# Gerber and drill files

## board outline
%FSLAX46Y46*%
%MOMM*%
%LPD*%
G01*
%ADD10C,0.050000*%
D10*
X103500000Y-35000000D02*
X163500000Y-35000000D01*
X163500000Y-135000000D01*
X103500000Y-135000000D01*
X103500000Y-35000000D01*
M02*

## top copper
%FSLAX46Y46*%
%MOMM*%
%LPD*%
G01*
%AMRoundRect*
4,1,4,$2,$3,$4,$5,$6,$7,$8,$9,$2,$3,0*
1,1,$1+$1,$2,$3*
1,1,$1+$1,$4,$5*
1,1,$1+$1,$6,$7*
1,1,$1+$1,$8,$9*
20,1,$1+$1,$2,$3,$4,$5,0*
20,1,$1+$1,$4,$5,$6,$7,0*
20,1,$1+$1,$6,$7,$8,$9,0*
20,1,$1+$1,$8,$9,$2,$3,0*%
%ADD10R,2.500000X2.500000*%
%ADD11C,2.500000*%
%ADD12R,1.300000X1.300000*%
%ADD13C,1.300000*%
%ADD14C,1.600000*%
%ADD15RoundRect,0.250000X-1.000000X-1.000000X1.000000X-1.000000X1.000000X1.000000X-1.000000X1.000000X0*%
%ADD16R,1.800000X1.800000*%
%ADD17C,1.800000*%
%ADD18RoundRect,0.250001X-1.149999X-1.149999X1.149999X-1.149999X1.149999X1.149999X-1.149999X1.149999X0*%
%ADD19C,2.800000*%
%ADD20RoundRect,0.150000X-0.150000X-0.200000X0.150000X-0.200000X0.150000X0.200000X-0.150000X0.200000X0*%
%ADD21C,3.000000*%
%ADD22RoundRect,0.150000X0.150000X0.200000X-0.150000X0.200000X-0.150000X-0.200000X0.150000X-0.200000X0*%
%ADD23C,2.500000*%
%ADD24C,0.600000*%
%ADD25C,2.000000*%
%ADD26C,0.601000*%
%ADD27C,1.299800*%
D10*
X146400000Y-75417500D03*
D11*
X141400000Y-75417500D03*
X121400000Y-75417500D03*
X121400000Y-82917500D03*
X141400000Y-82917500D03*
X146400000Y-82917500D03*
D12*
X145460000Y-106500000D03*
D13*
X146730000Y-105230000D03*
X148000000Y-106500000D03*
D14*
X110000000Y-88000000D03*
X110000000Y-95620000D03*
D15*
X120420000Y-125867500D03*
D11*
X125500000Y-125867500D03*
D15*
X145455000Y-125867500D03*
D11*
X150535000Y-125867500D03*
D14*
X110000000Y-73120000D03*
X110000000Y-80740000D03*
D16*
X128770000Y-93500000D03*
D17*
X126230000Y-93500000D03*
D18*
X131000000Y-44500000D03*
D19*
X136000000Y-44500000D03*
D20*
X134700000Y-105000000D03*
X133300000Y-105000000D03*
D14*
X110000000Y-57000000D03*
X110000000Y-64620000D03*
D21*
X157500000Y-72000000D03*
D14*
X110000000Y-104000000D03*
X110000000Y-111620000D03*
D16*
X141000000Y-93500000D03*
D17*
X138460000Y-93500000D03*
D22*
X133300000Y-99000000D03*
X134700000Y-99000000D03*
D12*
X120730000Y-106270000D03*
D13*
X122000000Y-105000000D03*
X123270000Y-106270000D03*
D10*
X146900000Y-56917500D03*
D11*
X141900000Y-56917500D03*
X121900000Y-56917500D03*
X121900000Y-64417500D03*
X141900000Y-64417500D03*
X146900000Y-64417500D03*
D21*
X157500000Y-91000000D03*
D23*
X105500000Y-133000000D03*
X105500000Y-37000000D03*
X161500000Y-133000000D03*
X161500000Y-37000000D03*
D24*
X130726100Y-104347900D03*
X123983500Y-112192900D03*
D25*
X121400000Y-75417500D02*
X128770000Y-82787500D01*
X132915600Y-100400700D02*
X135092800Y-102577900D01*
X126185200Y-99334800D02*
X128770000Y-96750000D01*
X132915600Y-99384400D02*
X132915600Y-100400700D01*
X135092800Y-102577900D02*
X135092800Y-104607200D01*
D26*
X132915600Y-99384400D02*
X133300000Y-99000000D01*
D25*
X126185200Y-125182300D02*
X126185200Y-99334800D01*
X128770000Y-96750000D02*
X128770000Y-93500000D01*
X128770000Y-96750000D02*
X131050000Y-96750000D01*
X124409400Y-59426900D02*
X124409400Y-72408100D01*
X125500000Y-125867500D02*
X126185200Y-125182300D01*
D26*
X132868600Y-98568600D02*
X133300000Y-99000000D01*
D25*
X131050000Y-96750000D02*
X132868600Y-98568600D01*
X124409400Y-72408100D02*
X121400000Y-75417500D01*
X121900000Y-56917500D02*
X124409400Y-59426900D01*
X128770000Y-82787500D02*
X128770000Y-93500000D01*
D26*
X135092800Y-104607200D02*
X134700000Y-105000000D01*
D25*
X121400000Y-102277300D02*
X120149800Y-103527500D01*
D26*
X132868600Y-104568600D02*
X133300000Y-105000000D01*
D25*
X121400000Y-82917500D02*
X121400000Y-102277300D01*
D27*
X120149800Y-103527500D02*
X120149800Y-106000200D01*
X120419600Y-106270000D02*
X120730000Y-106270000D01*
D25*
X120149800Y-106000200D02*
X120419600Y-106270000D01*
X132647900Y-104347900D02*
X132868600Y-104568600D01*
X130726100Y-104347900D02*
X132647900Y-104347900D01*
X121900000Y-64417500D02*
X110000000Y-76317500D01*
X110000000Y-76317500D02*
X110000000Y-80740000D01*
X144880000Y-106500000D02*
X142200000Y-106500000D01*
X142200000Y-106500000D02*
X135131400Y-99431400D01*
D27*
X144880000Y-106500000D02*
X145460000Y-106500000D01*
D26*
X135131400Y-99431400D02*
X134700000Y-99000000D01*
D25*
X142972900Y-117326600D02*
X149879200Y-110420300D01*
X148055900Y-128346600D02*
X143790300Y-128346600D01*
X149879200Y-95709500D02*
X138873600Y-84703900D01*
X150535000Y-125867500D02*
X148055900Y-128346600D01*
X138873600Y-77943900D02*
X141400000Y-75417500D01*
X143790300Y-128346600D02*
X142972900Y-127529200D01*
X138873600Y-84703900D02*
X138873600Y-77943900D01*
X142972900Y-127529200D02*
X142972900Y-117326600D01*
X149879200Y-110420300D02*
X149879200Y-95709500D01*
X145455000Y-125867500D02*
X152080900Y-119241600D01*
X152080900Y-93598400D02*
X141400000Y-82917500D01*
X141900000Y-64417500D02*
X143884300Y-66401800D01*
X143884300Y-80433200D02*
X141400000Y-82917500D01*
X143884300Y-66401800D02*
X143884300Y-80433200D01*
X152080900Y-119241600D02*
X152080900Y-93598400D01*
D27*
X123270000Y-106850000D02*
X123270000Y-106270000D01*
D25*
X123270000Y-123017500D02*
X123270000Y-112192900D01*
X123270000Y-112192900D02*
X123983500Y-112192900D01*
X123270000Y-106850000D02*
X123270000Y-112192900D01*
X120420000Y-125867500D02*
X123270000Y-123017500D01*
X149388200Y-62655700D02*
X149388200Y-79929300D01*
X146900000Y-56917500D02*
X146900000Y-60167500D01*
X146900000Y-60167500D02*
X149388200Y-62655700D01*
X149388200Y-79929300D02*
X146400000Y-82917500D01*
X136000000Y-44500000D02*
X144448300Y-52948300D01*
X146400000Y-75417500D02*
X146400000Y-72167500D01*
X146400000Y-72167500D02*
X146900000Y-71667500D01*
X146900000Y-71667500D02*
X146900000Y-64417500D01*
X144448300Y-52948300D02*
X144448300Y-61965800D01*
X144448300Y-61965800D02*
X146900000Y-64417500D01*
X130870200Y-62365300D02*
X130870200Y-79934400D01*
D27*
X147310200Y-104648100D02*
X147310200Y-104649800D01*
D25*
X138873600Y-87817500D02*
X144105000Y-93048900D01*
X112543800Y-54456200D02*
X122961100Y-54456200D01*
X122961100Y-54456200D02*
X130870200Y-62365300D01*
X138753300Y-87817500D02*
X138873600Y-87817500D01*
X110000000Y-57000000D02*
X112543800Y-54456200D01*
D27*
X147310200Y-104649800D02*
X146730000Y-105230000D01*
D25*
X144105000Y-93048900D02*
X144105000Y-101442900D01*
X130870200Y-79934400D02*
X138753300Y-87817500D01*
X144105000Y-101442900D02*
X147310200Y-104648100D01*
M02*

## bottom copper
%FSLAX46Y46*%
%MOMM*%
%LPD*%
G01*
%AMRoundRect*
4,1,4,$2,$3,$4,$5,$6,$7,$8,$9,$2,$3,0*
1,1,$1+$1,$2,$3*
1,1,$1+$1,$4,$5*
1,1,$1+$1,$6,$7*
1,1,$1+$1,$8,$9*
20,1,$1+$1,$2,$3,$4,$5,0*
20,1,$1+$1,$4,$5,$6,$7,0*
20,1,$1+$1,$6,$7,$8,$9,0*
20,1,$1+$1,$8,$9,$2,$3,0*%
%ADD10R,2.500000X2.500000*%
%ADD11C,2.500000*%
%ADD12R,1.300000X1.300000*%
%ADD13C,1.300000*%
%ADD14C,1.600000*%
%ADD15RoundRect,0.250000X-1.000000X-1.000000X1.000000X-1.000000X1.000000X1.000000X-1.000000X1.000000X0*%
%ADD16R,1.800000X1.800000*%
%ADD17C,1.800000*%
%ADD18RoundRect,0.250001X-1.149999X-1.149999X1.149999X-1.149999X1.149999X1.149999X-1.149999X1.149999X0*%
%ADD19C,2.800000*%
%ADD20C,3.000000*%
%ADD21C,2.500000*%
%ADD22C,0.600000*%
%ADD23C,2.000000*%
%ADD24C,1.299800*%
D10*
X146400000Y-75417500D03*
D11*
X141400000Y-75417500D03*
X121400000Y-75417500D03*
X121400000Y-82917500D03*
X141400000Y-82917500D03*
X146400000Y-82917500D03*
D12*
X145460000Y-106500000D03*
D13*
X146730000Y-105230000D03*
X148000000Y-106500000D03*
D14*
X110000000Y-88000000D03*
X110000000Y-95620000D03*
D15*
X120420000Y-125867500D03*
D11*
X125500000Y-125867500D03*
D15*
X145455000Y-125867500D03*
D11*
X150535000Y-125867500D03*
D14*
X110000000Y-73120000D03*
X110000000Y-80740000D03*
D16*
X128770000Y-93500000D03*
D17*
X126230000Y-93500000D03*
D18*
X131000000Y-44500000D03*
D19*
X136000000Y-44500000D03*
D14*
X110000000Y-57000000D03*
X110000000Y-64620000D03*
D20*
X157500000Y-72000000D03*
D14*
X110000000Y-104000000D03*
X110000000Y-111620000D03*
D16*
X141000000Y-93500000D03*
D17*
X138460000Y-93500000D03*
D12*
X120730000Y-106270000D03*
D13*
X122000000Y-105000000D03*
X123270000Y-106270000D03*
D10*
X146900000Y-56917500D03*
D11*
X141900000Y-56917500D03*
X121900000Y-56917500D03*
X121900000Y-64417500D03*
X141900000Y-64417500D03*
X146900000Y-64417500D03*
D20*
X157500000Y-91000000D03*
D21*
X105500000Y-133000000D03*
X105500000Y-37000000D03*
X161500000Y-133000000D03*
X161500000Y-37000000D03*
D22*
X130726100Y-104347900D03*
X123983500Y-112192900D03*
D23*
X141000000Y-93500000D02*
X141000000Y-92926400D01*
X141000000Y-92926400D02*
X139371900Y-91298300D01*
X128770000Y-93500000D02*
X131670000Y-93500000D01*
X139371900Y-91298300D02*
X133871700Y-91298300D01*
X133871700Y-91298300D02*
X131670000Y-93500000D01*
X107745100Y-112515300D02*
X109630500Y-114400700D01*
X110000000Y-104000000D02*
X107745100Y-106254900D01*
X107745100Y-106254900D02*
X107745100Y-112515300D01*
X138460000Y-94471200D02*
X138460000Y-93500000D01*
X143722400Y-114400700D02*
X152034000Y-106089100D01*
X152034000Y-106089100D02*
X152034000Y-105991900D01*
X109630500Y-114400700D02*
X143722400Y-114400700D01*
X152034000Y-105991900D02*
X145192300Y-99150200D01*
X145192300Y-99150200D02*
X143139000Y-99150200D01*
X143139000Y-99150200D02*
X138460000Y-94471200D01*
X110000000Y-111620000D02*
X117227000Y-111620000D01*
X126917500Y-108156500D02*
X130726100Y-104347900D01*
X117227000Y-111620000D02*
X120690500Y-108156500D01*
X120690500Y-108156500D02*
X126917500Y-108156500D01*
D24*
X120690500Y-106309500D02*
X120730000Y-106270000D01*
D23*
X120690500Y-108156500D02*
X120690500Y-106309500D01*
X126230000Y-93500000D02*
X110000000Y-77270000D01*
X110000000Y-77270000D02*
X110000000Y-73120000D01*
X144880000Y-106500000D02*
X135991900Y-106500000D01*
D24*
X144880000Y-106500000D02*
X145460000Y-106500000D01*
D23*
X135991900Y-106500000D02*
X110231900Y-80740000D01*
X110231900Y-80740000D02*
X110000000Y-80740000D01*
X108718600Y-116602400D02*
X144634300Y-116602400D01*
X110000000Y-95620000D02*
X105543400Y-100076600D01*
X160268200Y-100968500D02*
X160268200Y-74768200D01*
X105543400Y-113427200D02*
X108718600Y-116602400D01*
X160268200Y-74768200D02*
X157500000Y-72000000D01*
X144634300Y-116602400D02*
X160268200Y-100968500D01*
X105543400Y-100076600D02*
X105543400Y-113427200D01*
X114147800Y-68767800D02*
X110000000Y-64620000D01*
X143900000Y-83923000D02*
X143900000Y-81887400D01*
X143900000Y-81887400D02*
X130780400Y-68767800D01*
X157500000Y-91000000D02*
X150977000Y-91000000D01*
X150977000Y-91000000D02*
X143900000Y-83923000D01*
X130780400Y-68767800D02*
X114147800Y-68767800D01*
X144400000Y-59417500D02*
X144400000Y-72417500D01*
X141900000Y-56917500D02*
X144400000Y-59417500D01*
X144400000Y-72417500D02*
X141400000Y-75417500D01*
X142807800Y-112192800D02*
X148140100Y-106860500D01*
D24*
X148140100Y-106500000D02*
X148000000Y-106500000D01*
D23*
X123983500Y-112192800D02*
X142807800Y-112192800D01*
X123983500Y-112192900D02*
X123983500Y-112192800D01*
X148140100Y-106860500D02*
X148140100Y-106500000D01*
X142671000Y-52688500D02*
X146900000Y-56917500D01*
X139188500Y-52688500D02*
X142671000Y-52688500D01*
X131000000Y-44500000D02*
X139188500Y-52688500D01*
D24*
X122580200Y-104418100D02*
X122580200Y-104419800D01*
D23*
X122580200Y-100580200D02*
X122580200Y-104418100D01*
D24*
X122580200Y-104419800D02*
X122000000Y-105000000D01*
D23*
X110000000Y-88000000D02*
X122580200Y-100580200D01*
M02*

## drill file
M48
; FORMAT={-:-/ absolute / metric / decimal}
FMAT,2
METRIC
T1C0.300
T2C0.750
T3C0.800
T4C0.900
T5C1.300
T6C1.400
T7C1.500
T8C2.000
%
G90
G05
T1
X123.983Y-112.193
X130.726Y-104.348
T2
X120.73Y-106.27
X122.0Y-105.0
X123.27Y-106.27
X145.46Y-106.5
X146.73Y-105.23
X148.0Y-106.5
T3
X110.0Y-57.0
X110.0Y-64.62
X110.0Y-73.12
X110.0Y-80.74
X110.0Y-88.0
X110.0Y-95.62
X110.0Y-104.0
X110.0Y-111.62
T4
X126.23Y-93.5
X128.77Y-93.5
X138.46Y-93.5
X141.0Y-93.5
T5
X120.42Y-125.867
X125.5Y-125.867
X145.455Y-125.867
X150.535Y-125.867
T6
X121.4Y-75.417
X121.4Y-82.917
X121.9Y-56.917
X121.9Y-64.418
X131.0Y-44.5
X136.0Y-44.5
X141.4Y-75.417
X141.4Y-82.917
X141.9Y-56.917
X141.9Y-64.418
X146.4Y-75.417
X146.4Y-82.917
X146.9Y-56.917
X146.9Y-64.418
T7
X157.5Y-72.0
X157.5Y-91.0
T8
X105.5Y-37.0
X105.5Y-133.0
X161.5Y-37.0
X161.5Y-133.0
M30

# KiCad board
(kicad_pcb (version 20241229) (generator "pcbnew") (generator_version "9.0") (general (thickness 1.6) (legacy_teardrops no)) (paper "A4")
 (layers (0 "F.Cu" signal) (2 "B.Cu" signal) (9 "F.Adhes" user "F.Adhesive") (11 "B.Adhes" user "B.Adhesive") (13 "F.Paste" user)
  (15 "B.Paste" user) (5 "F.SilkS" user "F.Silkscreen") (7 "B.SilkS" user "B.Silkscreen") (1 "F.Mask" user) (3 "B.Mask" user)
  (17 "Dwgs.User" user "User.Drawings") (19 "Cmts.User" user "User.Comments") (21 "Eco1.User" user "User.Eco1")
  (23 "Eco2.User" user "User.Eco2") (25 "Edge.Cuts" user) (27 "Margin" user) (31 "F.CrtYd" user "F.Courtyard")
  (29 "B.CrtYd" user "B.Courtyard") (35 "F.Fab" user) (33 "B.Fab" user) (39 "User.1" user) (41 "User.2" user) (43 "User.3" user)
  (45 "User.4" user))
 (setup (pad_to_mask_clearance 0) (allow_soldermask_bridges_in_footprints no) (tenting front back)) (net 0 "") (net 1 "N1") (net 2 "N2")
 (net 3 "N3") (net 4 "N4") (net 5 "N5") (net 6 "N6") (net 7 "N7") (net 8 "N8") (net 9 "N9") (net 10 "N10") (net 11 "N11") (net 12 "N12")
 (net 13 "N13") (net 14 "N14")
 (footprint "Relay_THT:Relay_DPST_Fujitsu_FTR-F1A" (layer "F.Cu") (at 146.4 75.4175 -90)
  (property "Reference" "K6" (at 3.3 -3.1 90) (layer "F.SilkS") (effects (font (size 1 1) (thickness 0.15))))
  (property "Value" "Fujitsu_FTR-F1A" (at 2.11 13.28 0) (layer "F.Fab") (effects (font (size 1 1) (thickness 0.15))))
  (pad "1" thru_hole rect (at 0 0 180) (size 2.5 2.5) (drill 1.4) (layers "*.Cu" "*.Mask") (remove_unused_layers no) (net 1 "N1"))
  (pad "2" thru_hole circle (at 0 5 180) (size 2.5 2.5) (drill 1.4) (layers "*.Cu" "*.Mask") (remove_unused_layers no) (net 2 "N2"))
  (pad "4" thru_hole circle (at 0 25 180) (size 2.5 2.5) (drill 1.4) (layers "*.Cu" "*.Mask") (remove_unused_layers no) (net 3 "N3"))
  (pad "5" thru_hole circle (at 7.5 25 180) (size 2.5 2.5) (drill 1.4) (layers "*.Cu" "*.Mask") (remove_unused_layers no) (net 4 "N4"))
  (pad "7" thru_hole circle (at 7.5 5 180) (size 2.5 2.5) (drill 1.4) (layers "*.Cu" "*.Mask") (remove_unused_layers no) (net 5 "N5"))
  (pad "8" thru_hole circle (at 7.5 0 180) (size 2.5 2.5) (drill 1.4) (layers "*.Cu" "*.Mask") (remove_unused_layers no) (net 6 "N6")))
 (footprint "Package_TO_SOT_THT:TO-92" (layer "F.Cu") (at 145.46 106.5)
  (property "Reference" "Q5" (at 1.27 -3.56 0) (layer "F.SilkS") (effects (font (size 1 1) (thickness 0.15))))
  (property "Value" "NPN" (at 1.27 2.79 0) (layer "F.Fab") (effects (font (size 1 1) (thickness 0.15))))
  (pad "1" thru_hole rect (at 0 0) (size 1.3 1.3) (drill 0.75) (layers "*.Cu" "*.Mask") (remove_unused_layers no) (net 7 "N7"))
  (pad "2" thru_hole circle (at 1.27 -1.27) (size 1.3 1.3) (drill 0.75) (layers "*.Cu" "*.Mask") (remove_unused_layers no) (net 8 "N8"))
  (pad "3" thru_hole circle (at 2.54 0) (size 1.3 1.3) (drill 0.75) (layers "*.Cu" "*.Mask") (remove_unused_layers no) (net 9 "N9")))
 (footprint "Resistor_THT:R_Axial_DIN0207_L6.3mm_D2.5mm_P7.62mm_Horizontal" (layer "F.Cu") (at 110 88 -90)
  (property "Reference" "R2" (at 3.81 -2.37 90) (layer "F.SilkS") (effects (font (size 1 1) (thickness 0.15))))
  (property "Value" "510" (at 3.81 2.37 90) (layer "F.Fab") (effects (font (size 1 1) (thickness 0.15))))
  (pad "1" thru_hole circle (at 0 0 270) (size 1.6 1.6) (drill 0.8) (layers "*.Cu" "*.Mask") (remove_unused_layers no) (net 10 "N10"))
  (pad "2" thru_hole circle (at 7.62 0 270) (size 1.6 1.6) (drill 0.8) (layers "*.Cu" "*.Mask") (remove_unused_layers no) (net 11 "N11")))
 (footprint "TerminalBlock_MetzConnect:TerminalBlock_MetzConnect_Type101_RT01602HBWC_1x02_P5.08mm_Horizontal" (layer "F.Cu")
  (at 120.42 125.8675)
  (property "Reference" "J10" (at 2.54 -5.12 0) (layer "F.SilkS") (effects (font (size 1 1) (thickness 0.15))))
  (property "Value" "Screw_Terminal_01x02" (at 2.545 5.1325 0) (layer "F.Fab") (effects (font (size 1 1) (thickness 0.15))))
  (pad "1" thru_hole roundrect (at 0 0) (size 2.5 2.5) (drill 1.3) (layers "*.Cu" "*.Mask") (remove_unused_layers no) (roundrect_rratio 0.1)
   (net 9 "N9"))
  (pad "2" thru_hole circle (at 5.08 0) (size 2.5 2.5) (drill 1.3) (layers "*.Cu" "*.Mask") (remove_unused_layers no) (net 3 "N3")))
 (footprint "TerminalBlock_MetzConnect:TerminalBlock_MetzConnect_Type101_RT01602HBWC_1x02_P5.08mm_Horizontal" (layer "F.Cu")
  (at 145.455 125.8675)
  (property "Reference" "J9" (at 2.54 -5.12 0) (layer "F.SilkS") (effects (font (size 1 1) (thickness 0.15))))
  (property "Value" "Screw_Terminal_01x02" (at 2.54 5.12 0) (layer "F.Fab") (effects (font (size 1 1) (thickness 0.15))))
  (pad "1" thru_hole roundrect (at 0 0) (size 2.5 2.5) (drill 1.3) (layers "*.Cu" "*.Mask") (remove_unused_layers no) (roundrect_rratio 0.1)
   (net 5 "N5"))
  (pad "2" thru_hole circle (at 5.08 0) (size 2.5 2.5) (drill 1.3) (layers "*.Cu" "*.Mask") (remove_unused_layers no) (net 2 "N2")))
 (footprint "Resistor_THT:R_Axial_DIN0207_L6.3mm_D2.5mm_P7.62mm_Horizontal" (layer "F.Cu") (at 110 73.12 -90)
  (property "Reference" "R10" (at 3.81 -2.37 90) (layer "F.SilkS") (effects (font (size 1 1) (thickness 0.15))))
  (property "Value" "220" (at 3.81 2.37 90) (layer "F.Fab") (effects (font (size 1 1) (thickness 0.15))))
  (pad "1" thru_hole circle (at 0 0 270) (size 1.6 1.6) (drill 0.8) (layers "*.Cu" "*.Mask") (remove_unused_layers no) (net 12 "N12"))
  (pad "2" thru_hole circle (at 7.62 0 270) (size 1.6 1.6) (drill 0.8) (layers "*.Cu" "*.Mask") (remove_unused_layers no) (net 7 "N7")))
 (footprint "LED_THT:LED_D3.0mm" (layer "F.Cu") (at 128.77 93.5 180)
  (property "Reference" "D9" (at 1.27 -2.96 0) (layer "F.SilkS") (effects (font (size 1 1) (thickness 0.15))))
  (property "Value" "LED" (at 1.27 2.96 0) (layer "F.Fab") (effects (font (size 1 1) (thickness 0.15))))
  (pad "1" thru_hole rect (at 0 0 180) (size 1.8 1.8) (drill 0.9) (layers "*.Cu" "*.Mask") (remove_unused_layers no) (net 3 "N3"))
  (pad "2" thru_hole circle (at 2.54 0 180) (size 1.8 1.8) (drill 0.9) (layers "*.Cu" "*.Mask") (remove_unused_layers no) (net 12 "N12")))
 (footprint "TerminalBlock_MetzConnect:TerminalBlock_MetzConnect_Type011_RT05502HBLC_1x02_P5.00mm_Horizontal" (layer "F.Cu") (at 131 44.5)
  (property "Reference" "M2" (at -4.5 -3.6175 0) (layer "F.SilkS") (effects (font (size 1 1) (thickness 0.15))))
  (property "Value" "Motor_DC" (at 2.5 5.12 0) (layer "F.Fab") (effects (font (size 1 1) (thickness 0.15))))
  (pad "1" thru_hole roundrect (at 0 0) (size 2.8 2.8) (drill 1.4) (layers "*.Cu" "*.Mask") (remove_unused_layers no)
   (roundrect_rratio 0.089286) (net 6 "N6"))
  (pad "2" thru_hole circle (at 5 0) (size 2.8 2.8) (drill 1.4) (layers "*.Cu" "*.Mask") (remove_unused_layers no) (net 1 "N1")))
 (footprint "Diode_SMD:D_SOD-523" (layer "F.Cu") (at 134 105 180)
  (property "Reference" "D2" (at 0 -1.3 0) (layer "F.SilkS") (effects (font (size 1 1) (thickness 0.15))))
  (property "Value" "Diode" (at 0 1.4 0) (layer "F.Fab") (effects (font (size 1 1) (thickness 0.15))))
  (pad "1" smd roundrect (at -0.7 0) (size 0.6 0.7) (layers "F.Cu" "F.Mask" "F.Paste") (roundrect_rratio 0.25) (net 3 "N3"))
  (pad "2" smd roundrect (at 0.7 0) (size 0.6 0.7) (layers "F.Cu" "F.Mask" "F.Paste") (roundrect_rratio 0.25) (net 4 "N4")))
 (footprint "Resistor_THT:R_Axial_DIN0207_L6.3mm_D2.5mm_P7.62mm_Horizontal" (layer "F.Cu") (at 110 57 -90)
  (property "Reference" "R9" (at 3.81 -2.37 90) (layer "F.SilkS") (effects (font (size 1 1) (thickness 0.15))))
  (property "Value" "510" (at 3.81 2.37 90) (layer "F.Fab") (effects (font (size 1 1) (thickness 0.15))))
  (pad "1" thru_hole circle (at 0 0 270) (size 1.6 1.6) (drill 0.8) (layers "*.Cu" "*.Mask") (remove_unused_layers no) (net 8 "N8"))
  (pad "2" thru_hole circle (at 7.62 0 270) (size 1.6 1.6) (drill 0.8) (layers "*.Cu" "*.Mask") (remove_unused_layers no) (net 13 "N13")))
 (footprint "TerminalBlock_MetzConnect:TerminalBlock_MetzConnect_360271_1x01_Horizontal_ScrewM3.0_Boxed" (layer "F.Cu") (at 157.5 72 90)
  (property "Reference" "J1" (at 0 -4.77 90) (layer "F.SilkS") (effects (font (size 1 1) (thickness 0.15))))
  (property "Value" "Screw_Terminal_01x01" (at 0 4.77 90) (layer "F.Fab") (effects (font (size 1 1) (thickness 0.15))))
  (pad "1" thru_hole circle (at 0 0 90) (size 3 3) (drill 1.5) (layers "*.Cu" "*.Mask") (remove_unused_layers no) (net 11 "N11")))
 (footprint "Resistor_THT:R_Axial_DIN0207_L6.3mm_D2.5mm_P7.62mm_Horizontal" (layer "F.Cu") (at 110 104 -90)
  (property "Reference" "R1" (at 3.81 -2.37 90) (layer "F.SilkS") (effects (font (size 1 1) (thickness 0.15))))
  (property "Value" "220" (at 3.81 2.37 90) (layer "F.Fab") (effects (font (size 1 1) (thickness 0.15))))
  (pad "1" thru_hole circle (at 0 0 270) (size 1.6 1.6) (drill 0.8) (layers "*.Cu" "*.Mask") (remove_unused_layers no) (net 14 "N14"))
  (pad "2" thru_hole circle (at 7.62 0 270) (size 1.6 1.6) (drill 0.8) (layers "*.Cu" "*.Mask") (remove_unused_layers no) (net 4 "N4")))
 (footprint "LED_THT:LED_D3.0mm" (layer "F.Cu") (at 141 93.5 180)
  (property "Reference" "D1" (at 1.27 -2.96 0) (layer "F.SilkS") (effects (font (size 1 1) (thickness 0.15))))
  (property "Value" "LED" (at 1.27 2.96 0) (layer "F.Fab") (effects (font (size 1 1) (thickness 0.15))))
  (pad "1" thru_hole rect (at 0 0 180) (size 1.8 1.8) (drill 0.9) (layers "*.Cu" "*.Mask") (remove_unused_layers no) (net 3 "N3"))
  (pad "2" thru_hole circle (at 2.54 0 180) (size 1.8 1.8) (drill 0.9) (layers "*.Cu" "*.Mask") (remove_unused_layers no) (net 14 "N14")))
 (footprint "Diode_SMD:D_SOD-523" (layer "F.Cu") (at 134 99)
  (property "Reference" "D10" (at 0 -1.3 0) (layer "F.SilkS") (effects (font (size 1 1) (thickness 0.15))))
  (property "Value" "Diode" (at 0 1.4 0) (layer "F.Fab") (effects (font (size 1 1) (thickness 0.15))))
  (pad "1" smd roundrect (at -0.7 0 180) (size 0.6 0.7) (layers "F.Cu" "F.Mask" "F.Paste") (roundrect_rratio 0.25) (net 3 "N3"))
  (pad "2" smd roundrect (at 0.7 0 180) (size 0.6 0.7) (layers "F.Cu" "F.Mask" "F.Paste") (roundrect_rratio 0.25) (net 7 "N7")))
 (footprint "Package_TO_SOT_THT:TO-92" (layer "F.Cu") (at 120.73 106.27)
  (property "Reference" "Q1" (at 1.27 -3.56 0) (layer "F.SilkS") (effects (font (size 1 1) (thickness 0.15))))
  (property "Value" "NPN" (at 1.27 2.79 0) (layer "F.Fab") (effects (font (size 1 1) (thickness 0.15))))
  (pad "1" thru_hole rect (at 0 0) (size 1.3 1.3) (drill 0.75) (layers "*.Cu" "*.Mask") (remove_unused_layers no) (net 4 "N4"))
  (pad "2" thru_hole circle (at 1.27 -1.27) (size 1.3 1.3) (drill 0.75) (layers "*.Cu" "*.Mask") (remove_unused_layers no) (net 10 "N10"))
  (pad "3" thru_hole circle (at 2.54 0) (size 1.3 1.3) (drill 0.75) (layers "*.Cu" "*.Mask") (remove_unused_layers no) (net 9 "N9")))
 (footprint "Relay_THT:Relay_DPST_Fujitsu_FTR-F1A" (layer "F.Cu") (at 146.9 56.9175 -90)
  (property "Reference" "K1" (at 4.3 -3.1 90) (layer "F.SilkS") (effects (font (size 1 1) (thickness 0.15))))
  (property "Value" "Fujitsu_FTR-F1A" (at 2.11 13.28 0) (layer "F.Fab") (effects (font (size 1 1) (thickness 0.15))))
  (pad "1" thru_hole rect (at 0 0 180) (size 2.5 2.5) (drill 1.4) (layers "*.Cu" "*.Mask") (remove_unused_layers no) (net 6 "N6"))
  (pad "2" thru_hole circle (at 0 5 180) (size 2.5 2.5) (drill 1.4) (layers "*.Cu" "*.Mask") (remove_unused_layers no) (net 2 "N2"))
  (pad "4" thru_hole circle (at 0 25 180) (size 2.5 2.5) (drill 1.4) (layers "*.Cu" "*.Mask") (remove_unused_layers no) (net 3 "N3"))
  (pad "5" thru_hole circle (at 7.5 25 180) (size 2.5 2.5) (drill 1.4) (layers "*.Cu" "*.Mask") (remove_unused_layers no) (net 7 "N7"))
  (pad "7" thru_hole circle (at 7.5 5 180) (size 2.5 2.5) (drill 1.4) (layers "*.Cu" "*.Mask") (remove_unused_layers no) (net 5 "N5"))
  (pad "8" thru_hole circle (at 7.5 0 180) (size 2.5 2.5) (drill 1.4) (layers "*.Cu" "*.Mask") (remove_unused_layers no) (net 1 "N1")))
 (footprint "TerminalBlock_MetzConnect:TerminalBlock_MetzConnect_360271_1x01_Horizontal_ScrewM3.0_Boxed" (layer "F.Cu") (at 157.5 91 90)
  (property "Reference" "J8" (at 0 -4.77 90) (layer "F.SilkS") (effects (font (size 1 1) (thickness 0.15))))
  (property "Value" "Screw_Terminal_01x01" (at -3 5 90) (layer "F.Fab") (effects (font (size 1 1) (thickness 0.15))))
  (pad "1" thru_hole circle (at 0 0 90) (size 3 3) (drill 1.5) (layers "*.Cu" "*.Mask") (remove_unused_layers no) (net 13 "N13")))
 (gr_rect (start 103.5 35) (end 163.5 135) (stroke (width 0.05) (type default)) (fill no) (layer "Edge.Cuts"))
 (via (at 105.5 133) (size 2.5) (drill 2) (layers "F.Cu" "B.Cu") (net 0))
 (via (at 105.5 37) (size 2.5) (drill 2) (layers "F.Cu" "B.Cu") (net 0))
 (via (at 161.5 133) (size 2.5) (drill 2) (layers "F.Cu" "B.Cu") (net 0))
 (via (at 161.5 37) (size 2.5) (drill 2) (layers "F.Cu" "B.Cu") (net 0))
 (segment (start 121.4 75.4175) (end 128.77 82.7875) (width 2) (layer "F.Cu") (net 3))
 (segment (start 132.9156 100.4007) (end 135.0928 102.5779) (width 2) (layer "F.Cu") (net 3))
 (segment (start 126.1852 99.3348) (end 128.77 96.75) (width 2) (layer "F.Cu") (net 3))
 (segment (start 132.9156 99.3844) (end 132.9156 100.4007) (width 2) (layer "F.Cu") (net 3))
 (segment (start 135.0928 102.5779) (end 135.0928 104.6072) (width 2) (layer "F.Cu") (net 3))
 (segment (start 132.9156 99.3844) (end 133.3 99) (width 0.601) (layer "F.Cu") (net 3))
 (segment (start 126.1852 125.1823) (end 126.1852 99.3348) (width 2) (layer "F.Cu") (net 3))
 (segment (start 128.77 96.75) (end 128.77 93.5) (width 2) (layer "F.Cu") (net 3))
 (segment (start 128.77 96.75) (end 131.05 96.75) (width 2) (layer "F.Cu") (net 3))
 (segment (start 124.4094 59.4269) (end 124.4094 72.4081) (width 2) (layer "F.Cu") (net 3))
 (segment (start 125.5 125.8675) (end 126.1852 125.1823) (width 2) (layer "F.Cu") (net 3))
 (segment (start 132.8686 98.5686) (end 133.3 99) (width 0.601) (layer "F.Cu") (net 3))
 (segment (start 131.05 96.75) (end 132.8686 98.5686) (width 2) (layer "F.Cu") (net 3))
 (segment (start 124.4094 72.4081) (end 121.4 75.4175) (width 2) (layer "F.Cu") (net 3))
 (segment (start 121.9 56.9175) (end 124.4094 59.4269) (width 2) (layer "F.Cu") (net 3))
 (segment (start 128.77 82.7875) (end 128.77 93.5) (width 2) (layer "F.Cu") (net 3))
 (segment (start 135.0928 104.6072) (end 134.7 105) (width 0.601) (layer "F.Cu") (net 3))
 (segment (start 141 93.5) (end 141 92.9264) (width 2) (layer "B.Cu") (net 3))
 (segment (start 141 92.9264) (end 139.3719 91.2983) (width 2) (layer "B.Cu") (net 3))
 (segment (start 128.77 93.5) (end 131.67 93.5) (width 2) (layer "B.Cu") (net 3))
 (segment (start 139.3719 91.2983) (end 133.8717 91.2983) (width 2) (layer "B.Cu") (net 3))
 (segment (start 133.8717 91.2983) (end 131.67 93.5) (width 2) (layer "B.Cu") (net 3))
 (segment (start 107.7451 112.5153) (end 109.6305 114.4007) (width 2) (layer "B.Cu") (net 14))
 (segment (start 110 104) (end 107.7451 106.2549) (width 2) (layer "B.Cu") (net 14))
 (segment (start 107.7451 106.2549) (end 107.7451 112.5153) (width 2) (layer "B.Cu") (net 14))
 (segment (start 138.46 94.4712) (end 138.46 93.5) (width 2) (layer "B.Cu") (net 14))
 (segment (start 143.7224 114.4007) (end 152.034 106.0891) (width 2) (layer "B.Cu") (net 14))
 (segment (start 152.034 106.0891) (end 152.034 105.9919) (width 2) (layer "B.Cu") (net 14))
 (segment (start 109.6305 114.4007) (end 143.7224 114.4007) (width 2) (layer "B.Cu") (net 14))
 (segment (start 152.034 105.9919) (end 145.1923 99.1502) (width 2) (layer "B.Cu") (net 14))
 (segment (start 145.1923 99.1502) (end 143.139 99.1502) (width 2) (layer "B.Cu") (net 14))
 (segment (start 143.139 99.1502) (end 138.46 94.4712) (width 2) (layer "B.Cu") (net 14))
 (segment (start 121.4 102.2773) (end 120.1498 103.5275) (width 2) (layer "F.Cu") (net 4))
 (segment (start 132.8686 104.5686) (end 133.3 105) (width 0.601) (layer "F.Cu") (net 4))
 (segment (start 121.4 82.9175) (end 121.4 102.2773) (width 2) (layer "F.Cu") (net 4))
 (segment (start 120.1498 103.5275) (end 120.1498 106.0002) (width 1.2998) (layer "F.Cu") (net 4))
 (segment (start 120.4196 106.27) (end 120.73 106.27) (width 1.2998) (layer "F.Cu") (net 4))
 (segment (start 120.1498 106.0002) (end 120.4196 106.27) (width 2) (layer "F.Cu") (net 4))
 (segment (start 132.6479 104.3479) (end 132.8686 104.5686) (width 2) (layer "F.Cu") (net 4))
 (segment (start 130.7261 104.3479) (end 132.6479 104.3479) (width 2) (layer "F.Cu") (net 4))
 (via (at 130.7261 104.3479) (size 0.6) (drill 0.3) (layers "F.Cu" "B.Cu") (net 4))
 (segment (start 110 111.62) (end 117.227 111.62) (width 2) (layer "B.Cu") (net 4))
 (segment (start 126.9175 108.1565) (end 130.7261 104.3479) (width 2) (layer "B.Cu") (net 4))
 (segment (start 117.227 111.62) (end 120.6905 108.1565) (width 2) (layer "B.Cu") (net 4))
 (segment (start 120.6905 108.1565) (end 126.9175 108.1565) (width 2) (layer "B.Cu") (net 4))
 (segment (start 120.6905 106.3095) (end 120.73 106.27) (width 1.2998) (layer "B.Cu") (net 4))
 (segment (start 120.6905 108.1565) (end 120.6905 106.3095) (width 2) (layer "B.Cu") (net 4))
 (segment (start 126.23 93.5) (end 110 77.27) (width 2) (layer "B.Cu") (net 12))
 (segment (start 110 77.27) (end 110 73.12) (width 2) (layer "B.Cu") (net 12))
 (segment (start 121.9 64.4175) (end 110 76.3175) (width 2) (layer "F.Cu") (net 7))
 (segment (start 110 76.3175) (end 110 80.74) (width 2) (layer "F.Cu") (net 7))
 (segment (start 144.88 106.5) (end 142.2 106.5) (width 2) (layer "F.Cu") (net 7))
 (segment (start 142.2 106.5) (end 135.1314 99.4314) (width 2) (layer "F.Cu") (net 7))
 (segment (start 144.88 106.5) (end 145.46 106.5) (width 1.2998) (layer "F.Cu") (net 7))
 (segment (start 135.1314 99.4314) (end 134.7 99) (width 0.601) (layer "F.Cu") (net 7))
 (segment (start 144.88 106.5) (end 135.9919 106.5) (width 2) (layer "B.Cu") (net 7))
 (segment (start 144.88 106.5) (end 145.46 106.5) (width 1.2998) (layer "B.Cu") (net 7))
 (segment (start 135.9919 106.5) (end 110.2319 80.74) (width 2) (layer "B.Cu") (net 7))
 (segment (start 110.2319 80.74) (end 110 80.74) (width 2) (layer "B.Cu") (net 7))
 (segment (start 108.7186 116.6024) (end 144.6343 116.6024) (width 2) (layer "B.Cu") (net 11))
 (segment (start 110 95.62) (end 105.5434 100.0766) (width 2) (layer "B.Cu") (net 11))
 (segment (start 160.2682 100.9685) (end 160.2682 74.7682) (width 2) (layer "B.Cu") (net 11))
 (segment (start 105.5434 113.4272) (end 108.7186 116.6024) (width 2) (layer "B.Cu") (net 11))
 (segment (start 160.2682 74.7682) (end 157.5 72) (width 2) (layer "B.Cu") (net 11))
 (segment (start 144.6343 116.6024) (end 160.2682 100.9685) (width 2) (layer "B.Cu") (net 11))
 (segment (start 105.5434 100.0766) (end 105.5434 113.4272) (width 2) (layer "B.Cu") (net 11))
 (segment (start 114.1478 68.7678) (end 110 64.62) (width 2) (layer "B.Cu") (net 13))
 (segment (start 143.9 83.923) (end 143.9 81.8874) (width 2) (layer "B.Cu") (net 13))
 (segment (start 143.9 81.8874) (end 130.7804 68.7678) (width 2) (layer "B.Cu") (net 13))
 (segment (start 157.5 91) (end 150.977 91) (width 2) (layer "B.Cu") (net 13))
 (segment (start 150.977 91) (end 143.9 83.923) (width 2) (layer "B.Cu") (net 13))
 (segment (start 130.7804 68.7678) (end 114.1478 68.7678) (width 2) (layer "B.Cu") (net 13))
 (segment (start 142.9729 117.3266) (end 149.8792 110.4203) (width 2) (layer "F.Cu") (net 2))
 (segment (start 148.0559 128.3466) (end 143.7903 128.3466) (width 2) (layer "F.Cu") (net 2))
 (segment (start 149.8792 95.7095) (end 138.8736 84.7039) (width 2) (layer "F.Cu") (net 2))
 (segment (start 150.535 125.8675) (end 148.0559 128.3466) (width 2) (layer "F.Cu") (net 2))
 (segment (start 138.8736 77.9439) (end 141.4 75.4175) (width 2) (layer "F.Cu") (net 2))
 (segment (start 143.7903 128.3466) (end 142.9729 127.5292) (width 2) (layer "F.Cu") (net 2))
 (segment (start 138.8736 84.7039) (end 138.8736 77.9439) (width 2) (layer "F.Cu") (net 2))
 (segment (start 142.9729 127.5292) (end 142.9729 117.3266) (width 2) (layer "F.Cu") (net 2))
 (segment (start 149.8792 110.4203) (end 149.8792 95.7095) (width 2) (layer "F.Cu") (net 2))
 (segment (start 144.4 59.4175) (end 144.4 72.4175) (width 2) (layer "B.Cu") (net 2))
 (segment (start 141.9 56.9175) (end 144.4 59.4175) (width 2) (layer "B.Cu") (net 2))
 (segment (start 144.4 72.4175) (end 141.4 75.4175) (width 2) (layer "B.Cu") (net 2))
 (segment (start 145.455 125.8675) (end 152.0809 119.2416) (width 2) (layer "F.Cu") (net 5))
 (segment (start 152.0809 93.5984) (end 141.4 82.9175) (width 2) (layer "F.Cu") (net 5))
 (segment (start 141.9 64.4175) (end 143.8843 66.4018) (width 2) (layer "F.Cu") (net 5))
 (segment (start 143.8843 80.4332) (end 141.4 82.9175) (width 2) (layer "F.Cu") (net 5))
 (segment (start 143.8843 66.4018) (end 143.8843 80.4332) (width 2) (layer "F.Cu") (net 5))
 (segment (start 152.0809 119.2416) (end 152.0809 93.5984) (width 2) (layer "F.Cu") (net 5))
 (segment (start 123.27 106.85) (end 123.27 106.27) (width 1.2998) (layer "F.Cu") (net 9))
 (segment (start 123.27 123.0175) (end 123.27 112.1929) (width 2) (layer "F.Cu") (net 9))
 (segment (start 123.27 112.1929) (end 123.9835 112.1929) (width 2) (layer "F.Cu") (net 9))
 (segment (start 123.27 106.85) (end 123.27 112.1929) (width 2) (layer "F.Cu") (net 9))
 (segment (start 120.42 125.8675) (end 123.27 123.0175) (width 2) (layer "F.Cu") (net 9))
 (via (at 123.9835 112.1929) (size 0.6) (drill 0.3) (layers "F.Cu" "B.Cu") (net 9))
 (segment (start 142.8078 112.1928) (end 148.1401 106.8605) (width 2) (layer "B.Cu") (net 9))
 (segment (start 148.1401 106.5) (end 148 106.5) (width 1.2998) (layer "B.Cu") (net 9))
 (segment (start 123.9835 112.1928) (end 142.8078 112.1928) (width 2) (layer "B.Cu") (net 9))
 (segment (start 123.9835 112.1929) (end 123.9835 112.1928) (width 2) (layer "B.Cu") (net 9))
 (segment (start 148.1401 106.8605) (end 148.1401 106.5) (width 2) (layer "B.Cu") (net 9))
 (segment (start 149.3882 62.6557) (end 149.3882 79.9293) (width 2) (layer "F.Cu") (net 6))
 (segment (start 146.9 56.9175) (end 146.9 60.1675) (width 2) (layer "F.Cu") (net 6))
 (segment (start 146.9 60.1675) (end 149.3882 62.6557) (width 2) (layer "F.Cu") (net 6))
 (segment (start 149.3882 79.9293) (end 146.4 82.9175) (width 2) (layer "F.Cu") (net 6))
 (segment (start 142.671 52.6885) (end 146.9 56.9175) (width 2) (layer "B.Cu") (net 6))
 (segment (start 139.1885 52.6885) (end 142.671 52.6885) (width 2) (layer "B.Cu") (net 6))
 (segment (start 131 44.5) (end 139.1885 52.6885) (width 2) (layer "B.Cu") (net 6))
 (segment (start 136 44.5) (end 144.4483 52.9483) (width 2) (layer "F.Cu") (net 1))
 (segment (start 146.4 75.4175) (end 146.4 72.1675) (width 2) (layer "F.Cu") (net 1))
 (segment (start 146.4 72.1675) (end 146.9 71.6675) (width 2) (layer "F.Cu") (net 1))
 (segment (start 146.9 71.6675) (end 146.9 64.4175) (width 2) (layer "F.Cu") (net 1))
 (segment (start 144.4483 52.9483) (end 144.4483 61.9658) (width 2) (layer "F.Cu") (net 1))
 (segment (start 144.4483 61.9658) (end 146.9 64.4175) (width 2) (layer "F.Cu") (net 1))
 (segment (start 122.5802 104.4181) (end 122.5802 104.4198) (width 1.2998) (layer "B.Cu") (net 10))
 (segment (start 122.5802 100.5802) (end 122.5802 104.4181) (width 2) (layer "B.Cu") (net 10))
 (segment (start 122.5802 104.4198) (end 122 105) (width 1.2998) (layer "B.Cu") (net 10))
 (segment (start 110 88) (end 122.5802 100.5802) (width 2) (layer "B.Cu") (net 10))
 (segment (start 130.8702 62.3653) (end 130.8702 79.9344) (width 2) (layer "F.Cu") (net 8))
 (segment (start 147.3102 104.6481) (end 147.3102 104.6498) (width 1.2998) (layer "F.Cu") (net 8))
 (segment (start 138.8736 87.8175) (end 144.105 93.0489) (width 2) (layer "F.Cu") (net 8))
 (segment (start 112.5438 54.4562) (end 122.9611 54.4562) (width 2) (layer "F.Cu") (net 8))
 (segment (start 122.9611 54.4562) (end 130.8702 62.3653) (width 2) (layer "F.Cu") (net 8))
 (segment (start 138.7533 87.8175) (end 138.8736 87.8175) (width 2) (layer "F.Cu") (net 8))
 (segment (start 110 57) (end 112.5438 54.4562) (width 2) (layer "F.Cu") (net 8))
 (segment (start 147.3102 104.6498) (end 146.73 105.23) (width 1.2998) (layer "F.Cu") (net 8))
 (segment (start 144.105 93.0489) (end 144.105 101.4429) (width 2) (layer "F.Cu") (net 8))
 (segment (start 130.8702 79.9344) (end 138.7533 87.8175) (width 2) (layer "F.Cu") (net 8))
 (segment (start 144.105 101.4429) (end 147.3102 104.6481) (width 2) (layer "F.Cu") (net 8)))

